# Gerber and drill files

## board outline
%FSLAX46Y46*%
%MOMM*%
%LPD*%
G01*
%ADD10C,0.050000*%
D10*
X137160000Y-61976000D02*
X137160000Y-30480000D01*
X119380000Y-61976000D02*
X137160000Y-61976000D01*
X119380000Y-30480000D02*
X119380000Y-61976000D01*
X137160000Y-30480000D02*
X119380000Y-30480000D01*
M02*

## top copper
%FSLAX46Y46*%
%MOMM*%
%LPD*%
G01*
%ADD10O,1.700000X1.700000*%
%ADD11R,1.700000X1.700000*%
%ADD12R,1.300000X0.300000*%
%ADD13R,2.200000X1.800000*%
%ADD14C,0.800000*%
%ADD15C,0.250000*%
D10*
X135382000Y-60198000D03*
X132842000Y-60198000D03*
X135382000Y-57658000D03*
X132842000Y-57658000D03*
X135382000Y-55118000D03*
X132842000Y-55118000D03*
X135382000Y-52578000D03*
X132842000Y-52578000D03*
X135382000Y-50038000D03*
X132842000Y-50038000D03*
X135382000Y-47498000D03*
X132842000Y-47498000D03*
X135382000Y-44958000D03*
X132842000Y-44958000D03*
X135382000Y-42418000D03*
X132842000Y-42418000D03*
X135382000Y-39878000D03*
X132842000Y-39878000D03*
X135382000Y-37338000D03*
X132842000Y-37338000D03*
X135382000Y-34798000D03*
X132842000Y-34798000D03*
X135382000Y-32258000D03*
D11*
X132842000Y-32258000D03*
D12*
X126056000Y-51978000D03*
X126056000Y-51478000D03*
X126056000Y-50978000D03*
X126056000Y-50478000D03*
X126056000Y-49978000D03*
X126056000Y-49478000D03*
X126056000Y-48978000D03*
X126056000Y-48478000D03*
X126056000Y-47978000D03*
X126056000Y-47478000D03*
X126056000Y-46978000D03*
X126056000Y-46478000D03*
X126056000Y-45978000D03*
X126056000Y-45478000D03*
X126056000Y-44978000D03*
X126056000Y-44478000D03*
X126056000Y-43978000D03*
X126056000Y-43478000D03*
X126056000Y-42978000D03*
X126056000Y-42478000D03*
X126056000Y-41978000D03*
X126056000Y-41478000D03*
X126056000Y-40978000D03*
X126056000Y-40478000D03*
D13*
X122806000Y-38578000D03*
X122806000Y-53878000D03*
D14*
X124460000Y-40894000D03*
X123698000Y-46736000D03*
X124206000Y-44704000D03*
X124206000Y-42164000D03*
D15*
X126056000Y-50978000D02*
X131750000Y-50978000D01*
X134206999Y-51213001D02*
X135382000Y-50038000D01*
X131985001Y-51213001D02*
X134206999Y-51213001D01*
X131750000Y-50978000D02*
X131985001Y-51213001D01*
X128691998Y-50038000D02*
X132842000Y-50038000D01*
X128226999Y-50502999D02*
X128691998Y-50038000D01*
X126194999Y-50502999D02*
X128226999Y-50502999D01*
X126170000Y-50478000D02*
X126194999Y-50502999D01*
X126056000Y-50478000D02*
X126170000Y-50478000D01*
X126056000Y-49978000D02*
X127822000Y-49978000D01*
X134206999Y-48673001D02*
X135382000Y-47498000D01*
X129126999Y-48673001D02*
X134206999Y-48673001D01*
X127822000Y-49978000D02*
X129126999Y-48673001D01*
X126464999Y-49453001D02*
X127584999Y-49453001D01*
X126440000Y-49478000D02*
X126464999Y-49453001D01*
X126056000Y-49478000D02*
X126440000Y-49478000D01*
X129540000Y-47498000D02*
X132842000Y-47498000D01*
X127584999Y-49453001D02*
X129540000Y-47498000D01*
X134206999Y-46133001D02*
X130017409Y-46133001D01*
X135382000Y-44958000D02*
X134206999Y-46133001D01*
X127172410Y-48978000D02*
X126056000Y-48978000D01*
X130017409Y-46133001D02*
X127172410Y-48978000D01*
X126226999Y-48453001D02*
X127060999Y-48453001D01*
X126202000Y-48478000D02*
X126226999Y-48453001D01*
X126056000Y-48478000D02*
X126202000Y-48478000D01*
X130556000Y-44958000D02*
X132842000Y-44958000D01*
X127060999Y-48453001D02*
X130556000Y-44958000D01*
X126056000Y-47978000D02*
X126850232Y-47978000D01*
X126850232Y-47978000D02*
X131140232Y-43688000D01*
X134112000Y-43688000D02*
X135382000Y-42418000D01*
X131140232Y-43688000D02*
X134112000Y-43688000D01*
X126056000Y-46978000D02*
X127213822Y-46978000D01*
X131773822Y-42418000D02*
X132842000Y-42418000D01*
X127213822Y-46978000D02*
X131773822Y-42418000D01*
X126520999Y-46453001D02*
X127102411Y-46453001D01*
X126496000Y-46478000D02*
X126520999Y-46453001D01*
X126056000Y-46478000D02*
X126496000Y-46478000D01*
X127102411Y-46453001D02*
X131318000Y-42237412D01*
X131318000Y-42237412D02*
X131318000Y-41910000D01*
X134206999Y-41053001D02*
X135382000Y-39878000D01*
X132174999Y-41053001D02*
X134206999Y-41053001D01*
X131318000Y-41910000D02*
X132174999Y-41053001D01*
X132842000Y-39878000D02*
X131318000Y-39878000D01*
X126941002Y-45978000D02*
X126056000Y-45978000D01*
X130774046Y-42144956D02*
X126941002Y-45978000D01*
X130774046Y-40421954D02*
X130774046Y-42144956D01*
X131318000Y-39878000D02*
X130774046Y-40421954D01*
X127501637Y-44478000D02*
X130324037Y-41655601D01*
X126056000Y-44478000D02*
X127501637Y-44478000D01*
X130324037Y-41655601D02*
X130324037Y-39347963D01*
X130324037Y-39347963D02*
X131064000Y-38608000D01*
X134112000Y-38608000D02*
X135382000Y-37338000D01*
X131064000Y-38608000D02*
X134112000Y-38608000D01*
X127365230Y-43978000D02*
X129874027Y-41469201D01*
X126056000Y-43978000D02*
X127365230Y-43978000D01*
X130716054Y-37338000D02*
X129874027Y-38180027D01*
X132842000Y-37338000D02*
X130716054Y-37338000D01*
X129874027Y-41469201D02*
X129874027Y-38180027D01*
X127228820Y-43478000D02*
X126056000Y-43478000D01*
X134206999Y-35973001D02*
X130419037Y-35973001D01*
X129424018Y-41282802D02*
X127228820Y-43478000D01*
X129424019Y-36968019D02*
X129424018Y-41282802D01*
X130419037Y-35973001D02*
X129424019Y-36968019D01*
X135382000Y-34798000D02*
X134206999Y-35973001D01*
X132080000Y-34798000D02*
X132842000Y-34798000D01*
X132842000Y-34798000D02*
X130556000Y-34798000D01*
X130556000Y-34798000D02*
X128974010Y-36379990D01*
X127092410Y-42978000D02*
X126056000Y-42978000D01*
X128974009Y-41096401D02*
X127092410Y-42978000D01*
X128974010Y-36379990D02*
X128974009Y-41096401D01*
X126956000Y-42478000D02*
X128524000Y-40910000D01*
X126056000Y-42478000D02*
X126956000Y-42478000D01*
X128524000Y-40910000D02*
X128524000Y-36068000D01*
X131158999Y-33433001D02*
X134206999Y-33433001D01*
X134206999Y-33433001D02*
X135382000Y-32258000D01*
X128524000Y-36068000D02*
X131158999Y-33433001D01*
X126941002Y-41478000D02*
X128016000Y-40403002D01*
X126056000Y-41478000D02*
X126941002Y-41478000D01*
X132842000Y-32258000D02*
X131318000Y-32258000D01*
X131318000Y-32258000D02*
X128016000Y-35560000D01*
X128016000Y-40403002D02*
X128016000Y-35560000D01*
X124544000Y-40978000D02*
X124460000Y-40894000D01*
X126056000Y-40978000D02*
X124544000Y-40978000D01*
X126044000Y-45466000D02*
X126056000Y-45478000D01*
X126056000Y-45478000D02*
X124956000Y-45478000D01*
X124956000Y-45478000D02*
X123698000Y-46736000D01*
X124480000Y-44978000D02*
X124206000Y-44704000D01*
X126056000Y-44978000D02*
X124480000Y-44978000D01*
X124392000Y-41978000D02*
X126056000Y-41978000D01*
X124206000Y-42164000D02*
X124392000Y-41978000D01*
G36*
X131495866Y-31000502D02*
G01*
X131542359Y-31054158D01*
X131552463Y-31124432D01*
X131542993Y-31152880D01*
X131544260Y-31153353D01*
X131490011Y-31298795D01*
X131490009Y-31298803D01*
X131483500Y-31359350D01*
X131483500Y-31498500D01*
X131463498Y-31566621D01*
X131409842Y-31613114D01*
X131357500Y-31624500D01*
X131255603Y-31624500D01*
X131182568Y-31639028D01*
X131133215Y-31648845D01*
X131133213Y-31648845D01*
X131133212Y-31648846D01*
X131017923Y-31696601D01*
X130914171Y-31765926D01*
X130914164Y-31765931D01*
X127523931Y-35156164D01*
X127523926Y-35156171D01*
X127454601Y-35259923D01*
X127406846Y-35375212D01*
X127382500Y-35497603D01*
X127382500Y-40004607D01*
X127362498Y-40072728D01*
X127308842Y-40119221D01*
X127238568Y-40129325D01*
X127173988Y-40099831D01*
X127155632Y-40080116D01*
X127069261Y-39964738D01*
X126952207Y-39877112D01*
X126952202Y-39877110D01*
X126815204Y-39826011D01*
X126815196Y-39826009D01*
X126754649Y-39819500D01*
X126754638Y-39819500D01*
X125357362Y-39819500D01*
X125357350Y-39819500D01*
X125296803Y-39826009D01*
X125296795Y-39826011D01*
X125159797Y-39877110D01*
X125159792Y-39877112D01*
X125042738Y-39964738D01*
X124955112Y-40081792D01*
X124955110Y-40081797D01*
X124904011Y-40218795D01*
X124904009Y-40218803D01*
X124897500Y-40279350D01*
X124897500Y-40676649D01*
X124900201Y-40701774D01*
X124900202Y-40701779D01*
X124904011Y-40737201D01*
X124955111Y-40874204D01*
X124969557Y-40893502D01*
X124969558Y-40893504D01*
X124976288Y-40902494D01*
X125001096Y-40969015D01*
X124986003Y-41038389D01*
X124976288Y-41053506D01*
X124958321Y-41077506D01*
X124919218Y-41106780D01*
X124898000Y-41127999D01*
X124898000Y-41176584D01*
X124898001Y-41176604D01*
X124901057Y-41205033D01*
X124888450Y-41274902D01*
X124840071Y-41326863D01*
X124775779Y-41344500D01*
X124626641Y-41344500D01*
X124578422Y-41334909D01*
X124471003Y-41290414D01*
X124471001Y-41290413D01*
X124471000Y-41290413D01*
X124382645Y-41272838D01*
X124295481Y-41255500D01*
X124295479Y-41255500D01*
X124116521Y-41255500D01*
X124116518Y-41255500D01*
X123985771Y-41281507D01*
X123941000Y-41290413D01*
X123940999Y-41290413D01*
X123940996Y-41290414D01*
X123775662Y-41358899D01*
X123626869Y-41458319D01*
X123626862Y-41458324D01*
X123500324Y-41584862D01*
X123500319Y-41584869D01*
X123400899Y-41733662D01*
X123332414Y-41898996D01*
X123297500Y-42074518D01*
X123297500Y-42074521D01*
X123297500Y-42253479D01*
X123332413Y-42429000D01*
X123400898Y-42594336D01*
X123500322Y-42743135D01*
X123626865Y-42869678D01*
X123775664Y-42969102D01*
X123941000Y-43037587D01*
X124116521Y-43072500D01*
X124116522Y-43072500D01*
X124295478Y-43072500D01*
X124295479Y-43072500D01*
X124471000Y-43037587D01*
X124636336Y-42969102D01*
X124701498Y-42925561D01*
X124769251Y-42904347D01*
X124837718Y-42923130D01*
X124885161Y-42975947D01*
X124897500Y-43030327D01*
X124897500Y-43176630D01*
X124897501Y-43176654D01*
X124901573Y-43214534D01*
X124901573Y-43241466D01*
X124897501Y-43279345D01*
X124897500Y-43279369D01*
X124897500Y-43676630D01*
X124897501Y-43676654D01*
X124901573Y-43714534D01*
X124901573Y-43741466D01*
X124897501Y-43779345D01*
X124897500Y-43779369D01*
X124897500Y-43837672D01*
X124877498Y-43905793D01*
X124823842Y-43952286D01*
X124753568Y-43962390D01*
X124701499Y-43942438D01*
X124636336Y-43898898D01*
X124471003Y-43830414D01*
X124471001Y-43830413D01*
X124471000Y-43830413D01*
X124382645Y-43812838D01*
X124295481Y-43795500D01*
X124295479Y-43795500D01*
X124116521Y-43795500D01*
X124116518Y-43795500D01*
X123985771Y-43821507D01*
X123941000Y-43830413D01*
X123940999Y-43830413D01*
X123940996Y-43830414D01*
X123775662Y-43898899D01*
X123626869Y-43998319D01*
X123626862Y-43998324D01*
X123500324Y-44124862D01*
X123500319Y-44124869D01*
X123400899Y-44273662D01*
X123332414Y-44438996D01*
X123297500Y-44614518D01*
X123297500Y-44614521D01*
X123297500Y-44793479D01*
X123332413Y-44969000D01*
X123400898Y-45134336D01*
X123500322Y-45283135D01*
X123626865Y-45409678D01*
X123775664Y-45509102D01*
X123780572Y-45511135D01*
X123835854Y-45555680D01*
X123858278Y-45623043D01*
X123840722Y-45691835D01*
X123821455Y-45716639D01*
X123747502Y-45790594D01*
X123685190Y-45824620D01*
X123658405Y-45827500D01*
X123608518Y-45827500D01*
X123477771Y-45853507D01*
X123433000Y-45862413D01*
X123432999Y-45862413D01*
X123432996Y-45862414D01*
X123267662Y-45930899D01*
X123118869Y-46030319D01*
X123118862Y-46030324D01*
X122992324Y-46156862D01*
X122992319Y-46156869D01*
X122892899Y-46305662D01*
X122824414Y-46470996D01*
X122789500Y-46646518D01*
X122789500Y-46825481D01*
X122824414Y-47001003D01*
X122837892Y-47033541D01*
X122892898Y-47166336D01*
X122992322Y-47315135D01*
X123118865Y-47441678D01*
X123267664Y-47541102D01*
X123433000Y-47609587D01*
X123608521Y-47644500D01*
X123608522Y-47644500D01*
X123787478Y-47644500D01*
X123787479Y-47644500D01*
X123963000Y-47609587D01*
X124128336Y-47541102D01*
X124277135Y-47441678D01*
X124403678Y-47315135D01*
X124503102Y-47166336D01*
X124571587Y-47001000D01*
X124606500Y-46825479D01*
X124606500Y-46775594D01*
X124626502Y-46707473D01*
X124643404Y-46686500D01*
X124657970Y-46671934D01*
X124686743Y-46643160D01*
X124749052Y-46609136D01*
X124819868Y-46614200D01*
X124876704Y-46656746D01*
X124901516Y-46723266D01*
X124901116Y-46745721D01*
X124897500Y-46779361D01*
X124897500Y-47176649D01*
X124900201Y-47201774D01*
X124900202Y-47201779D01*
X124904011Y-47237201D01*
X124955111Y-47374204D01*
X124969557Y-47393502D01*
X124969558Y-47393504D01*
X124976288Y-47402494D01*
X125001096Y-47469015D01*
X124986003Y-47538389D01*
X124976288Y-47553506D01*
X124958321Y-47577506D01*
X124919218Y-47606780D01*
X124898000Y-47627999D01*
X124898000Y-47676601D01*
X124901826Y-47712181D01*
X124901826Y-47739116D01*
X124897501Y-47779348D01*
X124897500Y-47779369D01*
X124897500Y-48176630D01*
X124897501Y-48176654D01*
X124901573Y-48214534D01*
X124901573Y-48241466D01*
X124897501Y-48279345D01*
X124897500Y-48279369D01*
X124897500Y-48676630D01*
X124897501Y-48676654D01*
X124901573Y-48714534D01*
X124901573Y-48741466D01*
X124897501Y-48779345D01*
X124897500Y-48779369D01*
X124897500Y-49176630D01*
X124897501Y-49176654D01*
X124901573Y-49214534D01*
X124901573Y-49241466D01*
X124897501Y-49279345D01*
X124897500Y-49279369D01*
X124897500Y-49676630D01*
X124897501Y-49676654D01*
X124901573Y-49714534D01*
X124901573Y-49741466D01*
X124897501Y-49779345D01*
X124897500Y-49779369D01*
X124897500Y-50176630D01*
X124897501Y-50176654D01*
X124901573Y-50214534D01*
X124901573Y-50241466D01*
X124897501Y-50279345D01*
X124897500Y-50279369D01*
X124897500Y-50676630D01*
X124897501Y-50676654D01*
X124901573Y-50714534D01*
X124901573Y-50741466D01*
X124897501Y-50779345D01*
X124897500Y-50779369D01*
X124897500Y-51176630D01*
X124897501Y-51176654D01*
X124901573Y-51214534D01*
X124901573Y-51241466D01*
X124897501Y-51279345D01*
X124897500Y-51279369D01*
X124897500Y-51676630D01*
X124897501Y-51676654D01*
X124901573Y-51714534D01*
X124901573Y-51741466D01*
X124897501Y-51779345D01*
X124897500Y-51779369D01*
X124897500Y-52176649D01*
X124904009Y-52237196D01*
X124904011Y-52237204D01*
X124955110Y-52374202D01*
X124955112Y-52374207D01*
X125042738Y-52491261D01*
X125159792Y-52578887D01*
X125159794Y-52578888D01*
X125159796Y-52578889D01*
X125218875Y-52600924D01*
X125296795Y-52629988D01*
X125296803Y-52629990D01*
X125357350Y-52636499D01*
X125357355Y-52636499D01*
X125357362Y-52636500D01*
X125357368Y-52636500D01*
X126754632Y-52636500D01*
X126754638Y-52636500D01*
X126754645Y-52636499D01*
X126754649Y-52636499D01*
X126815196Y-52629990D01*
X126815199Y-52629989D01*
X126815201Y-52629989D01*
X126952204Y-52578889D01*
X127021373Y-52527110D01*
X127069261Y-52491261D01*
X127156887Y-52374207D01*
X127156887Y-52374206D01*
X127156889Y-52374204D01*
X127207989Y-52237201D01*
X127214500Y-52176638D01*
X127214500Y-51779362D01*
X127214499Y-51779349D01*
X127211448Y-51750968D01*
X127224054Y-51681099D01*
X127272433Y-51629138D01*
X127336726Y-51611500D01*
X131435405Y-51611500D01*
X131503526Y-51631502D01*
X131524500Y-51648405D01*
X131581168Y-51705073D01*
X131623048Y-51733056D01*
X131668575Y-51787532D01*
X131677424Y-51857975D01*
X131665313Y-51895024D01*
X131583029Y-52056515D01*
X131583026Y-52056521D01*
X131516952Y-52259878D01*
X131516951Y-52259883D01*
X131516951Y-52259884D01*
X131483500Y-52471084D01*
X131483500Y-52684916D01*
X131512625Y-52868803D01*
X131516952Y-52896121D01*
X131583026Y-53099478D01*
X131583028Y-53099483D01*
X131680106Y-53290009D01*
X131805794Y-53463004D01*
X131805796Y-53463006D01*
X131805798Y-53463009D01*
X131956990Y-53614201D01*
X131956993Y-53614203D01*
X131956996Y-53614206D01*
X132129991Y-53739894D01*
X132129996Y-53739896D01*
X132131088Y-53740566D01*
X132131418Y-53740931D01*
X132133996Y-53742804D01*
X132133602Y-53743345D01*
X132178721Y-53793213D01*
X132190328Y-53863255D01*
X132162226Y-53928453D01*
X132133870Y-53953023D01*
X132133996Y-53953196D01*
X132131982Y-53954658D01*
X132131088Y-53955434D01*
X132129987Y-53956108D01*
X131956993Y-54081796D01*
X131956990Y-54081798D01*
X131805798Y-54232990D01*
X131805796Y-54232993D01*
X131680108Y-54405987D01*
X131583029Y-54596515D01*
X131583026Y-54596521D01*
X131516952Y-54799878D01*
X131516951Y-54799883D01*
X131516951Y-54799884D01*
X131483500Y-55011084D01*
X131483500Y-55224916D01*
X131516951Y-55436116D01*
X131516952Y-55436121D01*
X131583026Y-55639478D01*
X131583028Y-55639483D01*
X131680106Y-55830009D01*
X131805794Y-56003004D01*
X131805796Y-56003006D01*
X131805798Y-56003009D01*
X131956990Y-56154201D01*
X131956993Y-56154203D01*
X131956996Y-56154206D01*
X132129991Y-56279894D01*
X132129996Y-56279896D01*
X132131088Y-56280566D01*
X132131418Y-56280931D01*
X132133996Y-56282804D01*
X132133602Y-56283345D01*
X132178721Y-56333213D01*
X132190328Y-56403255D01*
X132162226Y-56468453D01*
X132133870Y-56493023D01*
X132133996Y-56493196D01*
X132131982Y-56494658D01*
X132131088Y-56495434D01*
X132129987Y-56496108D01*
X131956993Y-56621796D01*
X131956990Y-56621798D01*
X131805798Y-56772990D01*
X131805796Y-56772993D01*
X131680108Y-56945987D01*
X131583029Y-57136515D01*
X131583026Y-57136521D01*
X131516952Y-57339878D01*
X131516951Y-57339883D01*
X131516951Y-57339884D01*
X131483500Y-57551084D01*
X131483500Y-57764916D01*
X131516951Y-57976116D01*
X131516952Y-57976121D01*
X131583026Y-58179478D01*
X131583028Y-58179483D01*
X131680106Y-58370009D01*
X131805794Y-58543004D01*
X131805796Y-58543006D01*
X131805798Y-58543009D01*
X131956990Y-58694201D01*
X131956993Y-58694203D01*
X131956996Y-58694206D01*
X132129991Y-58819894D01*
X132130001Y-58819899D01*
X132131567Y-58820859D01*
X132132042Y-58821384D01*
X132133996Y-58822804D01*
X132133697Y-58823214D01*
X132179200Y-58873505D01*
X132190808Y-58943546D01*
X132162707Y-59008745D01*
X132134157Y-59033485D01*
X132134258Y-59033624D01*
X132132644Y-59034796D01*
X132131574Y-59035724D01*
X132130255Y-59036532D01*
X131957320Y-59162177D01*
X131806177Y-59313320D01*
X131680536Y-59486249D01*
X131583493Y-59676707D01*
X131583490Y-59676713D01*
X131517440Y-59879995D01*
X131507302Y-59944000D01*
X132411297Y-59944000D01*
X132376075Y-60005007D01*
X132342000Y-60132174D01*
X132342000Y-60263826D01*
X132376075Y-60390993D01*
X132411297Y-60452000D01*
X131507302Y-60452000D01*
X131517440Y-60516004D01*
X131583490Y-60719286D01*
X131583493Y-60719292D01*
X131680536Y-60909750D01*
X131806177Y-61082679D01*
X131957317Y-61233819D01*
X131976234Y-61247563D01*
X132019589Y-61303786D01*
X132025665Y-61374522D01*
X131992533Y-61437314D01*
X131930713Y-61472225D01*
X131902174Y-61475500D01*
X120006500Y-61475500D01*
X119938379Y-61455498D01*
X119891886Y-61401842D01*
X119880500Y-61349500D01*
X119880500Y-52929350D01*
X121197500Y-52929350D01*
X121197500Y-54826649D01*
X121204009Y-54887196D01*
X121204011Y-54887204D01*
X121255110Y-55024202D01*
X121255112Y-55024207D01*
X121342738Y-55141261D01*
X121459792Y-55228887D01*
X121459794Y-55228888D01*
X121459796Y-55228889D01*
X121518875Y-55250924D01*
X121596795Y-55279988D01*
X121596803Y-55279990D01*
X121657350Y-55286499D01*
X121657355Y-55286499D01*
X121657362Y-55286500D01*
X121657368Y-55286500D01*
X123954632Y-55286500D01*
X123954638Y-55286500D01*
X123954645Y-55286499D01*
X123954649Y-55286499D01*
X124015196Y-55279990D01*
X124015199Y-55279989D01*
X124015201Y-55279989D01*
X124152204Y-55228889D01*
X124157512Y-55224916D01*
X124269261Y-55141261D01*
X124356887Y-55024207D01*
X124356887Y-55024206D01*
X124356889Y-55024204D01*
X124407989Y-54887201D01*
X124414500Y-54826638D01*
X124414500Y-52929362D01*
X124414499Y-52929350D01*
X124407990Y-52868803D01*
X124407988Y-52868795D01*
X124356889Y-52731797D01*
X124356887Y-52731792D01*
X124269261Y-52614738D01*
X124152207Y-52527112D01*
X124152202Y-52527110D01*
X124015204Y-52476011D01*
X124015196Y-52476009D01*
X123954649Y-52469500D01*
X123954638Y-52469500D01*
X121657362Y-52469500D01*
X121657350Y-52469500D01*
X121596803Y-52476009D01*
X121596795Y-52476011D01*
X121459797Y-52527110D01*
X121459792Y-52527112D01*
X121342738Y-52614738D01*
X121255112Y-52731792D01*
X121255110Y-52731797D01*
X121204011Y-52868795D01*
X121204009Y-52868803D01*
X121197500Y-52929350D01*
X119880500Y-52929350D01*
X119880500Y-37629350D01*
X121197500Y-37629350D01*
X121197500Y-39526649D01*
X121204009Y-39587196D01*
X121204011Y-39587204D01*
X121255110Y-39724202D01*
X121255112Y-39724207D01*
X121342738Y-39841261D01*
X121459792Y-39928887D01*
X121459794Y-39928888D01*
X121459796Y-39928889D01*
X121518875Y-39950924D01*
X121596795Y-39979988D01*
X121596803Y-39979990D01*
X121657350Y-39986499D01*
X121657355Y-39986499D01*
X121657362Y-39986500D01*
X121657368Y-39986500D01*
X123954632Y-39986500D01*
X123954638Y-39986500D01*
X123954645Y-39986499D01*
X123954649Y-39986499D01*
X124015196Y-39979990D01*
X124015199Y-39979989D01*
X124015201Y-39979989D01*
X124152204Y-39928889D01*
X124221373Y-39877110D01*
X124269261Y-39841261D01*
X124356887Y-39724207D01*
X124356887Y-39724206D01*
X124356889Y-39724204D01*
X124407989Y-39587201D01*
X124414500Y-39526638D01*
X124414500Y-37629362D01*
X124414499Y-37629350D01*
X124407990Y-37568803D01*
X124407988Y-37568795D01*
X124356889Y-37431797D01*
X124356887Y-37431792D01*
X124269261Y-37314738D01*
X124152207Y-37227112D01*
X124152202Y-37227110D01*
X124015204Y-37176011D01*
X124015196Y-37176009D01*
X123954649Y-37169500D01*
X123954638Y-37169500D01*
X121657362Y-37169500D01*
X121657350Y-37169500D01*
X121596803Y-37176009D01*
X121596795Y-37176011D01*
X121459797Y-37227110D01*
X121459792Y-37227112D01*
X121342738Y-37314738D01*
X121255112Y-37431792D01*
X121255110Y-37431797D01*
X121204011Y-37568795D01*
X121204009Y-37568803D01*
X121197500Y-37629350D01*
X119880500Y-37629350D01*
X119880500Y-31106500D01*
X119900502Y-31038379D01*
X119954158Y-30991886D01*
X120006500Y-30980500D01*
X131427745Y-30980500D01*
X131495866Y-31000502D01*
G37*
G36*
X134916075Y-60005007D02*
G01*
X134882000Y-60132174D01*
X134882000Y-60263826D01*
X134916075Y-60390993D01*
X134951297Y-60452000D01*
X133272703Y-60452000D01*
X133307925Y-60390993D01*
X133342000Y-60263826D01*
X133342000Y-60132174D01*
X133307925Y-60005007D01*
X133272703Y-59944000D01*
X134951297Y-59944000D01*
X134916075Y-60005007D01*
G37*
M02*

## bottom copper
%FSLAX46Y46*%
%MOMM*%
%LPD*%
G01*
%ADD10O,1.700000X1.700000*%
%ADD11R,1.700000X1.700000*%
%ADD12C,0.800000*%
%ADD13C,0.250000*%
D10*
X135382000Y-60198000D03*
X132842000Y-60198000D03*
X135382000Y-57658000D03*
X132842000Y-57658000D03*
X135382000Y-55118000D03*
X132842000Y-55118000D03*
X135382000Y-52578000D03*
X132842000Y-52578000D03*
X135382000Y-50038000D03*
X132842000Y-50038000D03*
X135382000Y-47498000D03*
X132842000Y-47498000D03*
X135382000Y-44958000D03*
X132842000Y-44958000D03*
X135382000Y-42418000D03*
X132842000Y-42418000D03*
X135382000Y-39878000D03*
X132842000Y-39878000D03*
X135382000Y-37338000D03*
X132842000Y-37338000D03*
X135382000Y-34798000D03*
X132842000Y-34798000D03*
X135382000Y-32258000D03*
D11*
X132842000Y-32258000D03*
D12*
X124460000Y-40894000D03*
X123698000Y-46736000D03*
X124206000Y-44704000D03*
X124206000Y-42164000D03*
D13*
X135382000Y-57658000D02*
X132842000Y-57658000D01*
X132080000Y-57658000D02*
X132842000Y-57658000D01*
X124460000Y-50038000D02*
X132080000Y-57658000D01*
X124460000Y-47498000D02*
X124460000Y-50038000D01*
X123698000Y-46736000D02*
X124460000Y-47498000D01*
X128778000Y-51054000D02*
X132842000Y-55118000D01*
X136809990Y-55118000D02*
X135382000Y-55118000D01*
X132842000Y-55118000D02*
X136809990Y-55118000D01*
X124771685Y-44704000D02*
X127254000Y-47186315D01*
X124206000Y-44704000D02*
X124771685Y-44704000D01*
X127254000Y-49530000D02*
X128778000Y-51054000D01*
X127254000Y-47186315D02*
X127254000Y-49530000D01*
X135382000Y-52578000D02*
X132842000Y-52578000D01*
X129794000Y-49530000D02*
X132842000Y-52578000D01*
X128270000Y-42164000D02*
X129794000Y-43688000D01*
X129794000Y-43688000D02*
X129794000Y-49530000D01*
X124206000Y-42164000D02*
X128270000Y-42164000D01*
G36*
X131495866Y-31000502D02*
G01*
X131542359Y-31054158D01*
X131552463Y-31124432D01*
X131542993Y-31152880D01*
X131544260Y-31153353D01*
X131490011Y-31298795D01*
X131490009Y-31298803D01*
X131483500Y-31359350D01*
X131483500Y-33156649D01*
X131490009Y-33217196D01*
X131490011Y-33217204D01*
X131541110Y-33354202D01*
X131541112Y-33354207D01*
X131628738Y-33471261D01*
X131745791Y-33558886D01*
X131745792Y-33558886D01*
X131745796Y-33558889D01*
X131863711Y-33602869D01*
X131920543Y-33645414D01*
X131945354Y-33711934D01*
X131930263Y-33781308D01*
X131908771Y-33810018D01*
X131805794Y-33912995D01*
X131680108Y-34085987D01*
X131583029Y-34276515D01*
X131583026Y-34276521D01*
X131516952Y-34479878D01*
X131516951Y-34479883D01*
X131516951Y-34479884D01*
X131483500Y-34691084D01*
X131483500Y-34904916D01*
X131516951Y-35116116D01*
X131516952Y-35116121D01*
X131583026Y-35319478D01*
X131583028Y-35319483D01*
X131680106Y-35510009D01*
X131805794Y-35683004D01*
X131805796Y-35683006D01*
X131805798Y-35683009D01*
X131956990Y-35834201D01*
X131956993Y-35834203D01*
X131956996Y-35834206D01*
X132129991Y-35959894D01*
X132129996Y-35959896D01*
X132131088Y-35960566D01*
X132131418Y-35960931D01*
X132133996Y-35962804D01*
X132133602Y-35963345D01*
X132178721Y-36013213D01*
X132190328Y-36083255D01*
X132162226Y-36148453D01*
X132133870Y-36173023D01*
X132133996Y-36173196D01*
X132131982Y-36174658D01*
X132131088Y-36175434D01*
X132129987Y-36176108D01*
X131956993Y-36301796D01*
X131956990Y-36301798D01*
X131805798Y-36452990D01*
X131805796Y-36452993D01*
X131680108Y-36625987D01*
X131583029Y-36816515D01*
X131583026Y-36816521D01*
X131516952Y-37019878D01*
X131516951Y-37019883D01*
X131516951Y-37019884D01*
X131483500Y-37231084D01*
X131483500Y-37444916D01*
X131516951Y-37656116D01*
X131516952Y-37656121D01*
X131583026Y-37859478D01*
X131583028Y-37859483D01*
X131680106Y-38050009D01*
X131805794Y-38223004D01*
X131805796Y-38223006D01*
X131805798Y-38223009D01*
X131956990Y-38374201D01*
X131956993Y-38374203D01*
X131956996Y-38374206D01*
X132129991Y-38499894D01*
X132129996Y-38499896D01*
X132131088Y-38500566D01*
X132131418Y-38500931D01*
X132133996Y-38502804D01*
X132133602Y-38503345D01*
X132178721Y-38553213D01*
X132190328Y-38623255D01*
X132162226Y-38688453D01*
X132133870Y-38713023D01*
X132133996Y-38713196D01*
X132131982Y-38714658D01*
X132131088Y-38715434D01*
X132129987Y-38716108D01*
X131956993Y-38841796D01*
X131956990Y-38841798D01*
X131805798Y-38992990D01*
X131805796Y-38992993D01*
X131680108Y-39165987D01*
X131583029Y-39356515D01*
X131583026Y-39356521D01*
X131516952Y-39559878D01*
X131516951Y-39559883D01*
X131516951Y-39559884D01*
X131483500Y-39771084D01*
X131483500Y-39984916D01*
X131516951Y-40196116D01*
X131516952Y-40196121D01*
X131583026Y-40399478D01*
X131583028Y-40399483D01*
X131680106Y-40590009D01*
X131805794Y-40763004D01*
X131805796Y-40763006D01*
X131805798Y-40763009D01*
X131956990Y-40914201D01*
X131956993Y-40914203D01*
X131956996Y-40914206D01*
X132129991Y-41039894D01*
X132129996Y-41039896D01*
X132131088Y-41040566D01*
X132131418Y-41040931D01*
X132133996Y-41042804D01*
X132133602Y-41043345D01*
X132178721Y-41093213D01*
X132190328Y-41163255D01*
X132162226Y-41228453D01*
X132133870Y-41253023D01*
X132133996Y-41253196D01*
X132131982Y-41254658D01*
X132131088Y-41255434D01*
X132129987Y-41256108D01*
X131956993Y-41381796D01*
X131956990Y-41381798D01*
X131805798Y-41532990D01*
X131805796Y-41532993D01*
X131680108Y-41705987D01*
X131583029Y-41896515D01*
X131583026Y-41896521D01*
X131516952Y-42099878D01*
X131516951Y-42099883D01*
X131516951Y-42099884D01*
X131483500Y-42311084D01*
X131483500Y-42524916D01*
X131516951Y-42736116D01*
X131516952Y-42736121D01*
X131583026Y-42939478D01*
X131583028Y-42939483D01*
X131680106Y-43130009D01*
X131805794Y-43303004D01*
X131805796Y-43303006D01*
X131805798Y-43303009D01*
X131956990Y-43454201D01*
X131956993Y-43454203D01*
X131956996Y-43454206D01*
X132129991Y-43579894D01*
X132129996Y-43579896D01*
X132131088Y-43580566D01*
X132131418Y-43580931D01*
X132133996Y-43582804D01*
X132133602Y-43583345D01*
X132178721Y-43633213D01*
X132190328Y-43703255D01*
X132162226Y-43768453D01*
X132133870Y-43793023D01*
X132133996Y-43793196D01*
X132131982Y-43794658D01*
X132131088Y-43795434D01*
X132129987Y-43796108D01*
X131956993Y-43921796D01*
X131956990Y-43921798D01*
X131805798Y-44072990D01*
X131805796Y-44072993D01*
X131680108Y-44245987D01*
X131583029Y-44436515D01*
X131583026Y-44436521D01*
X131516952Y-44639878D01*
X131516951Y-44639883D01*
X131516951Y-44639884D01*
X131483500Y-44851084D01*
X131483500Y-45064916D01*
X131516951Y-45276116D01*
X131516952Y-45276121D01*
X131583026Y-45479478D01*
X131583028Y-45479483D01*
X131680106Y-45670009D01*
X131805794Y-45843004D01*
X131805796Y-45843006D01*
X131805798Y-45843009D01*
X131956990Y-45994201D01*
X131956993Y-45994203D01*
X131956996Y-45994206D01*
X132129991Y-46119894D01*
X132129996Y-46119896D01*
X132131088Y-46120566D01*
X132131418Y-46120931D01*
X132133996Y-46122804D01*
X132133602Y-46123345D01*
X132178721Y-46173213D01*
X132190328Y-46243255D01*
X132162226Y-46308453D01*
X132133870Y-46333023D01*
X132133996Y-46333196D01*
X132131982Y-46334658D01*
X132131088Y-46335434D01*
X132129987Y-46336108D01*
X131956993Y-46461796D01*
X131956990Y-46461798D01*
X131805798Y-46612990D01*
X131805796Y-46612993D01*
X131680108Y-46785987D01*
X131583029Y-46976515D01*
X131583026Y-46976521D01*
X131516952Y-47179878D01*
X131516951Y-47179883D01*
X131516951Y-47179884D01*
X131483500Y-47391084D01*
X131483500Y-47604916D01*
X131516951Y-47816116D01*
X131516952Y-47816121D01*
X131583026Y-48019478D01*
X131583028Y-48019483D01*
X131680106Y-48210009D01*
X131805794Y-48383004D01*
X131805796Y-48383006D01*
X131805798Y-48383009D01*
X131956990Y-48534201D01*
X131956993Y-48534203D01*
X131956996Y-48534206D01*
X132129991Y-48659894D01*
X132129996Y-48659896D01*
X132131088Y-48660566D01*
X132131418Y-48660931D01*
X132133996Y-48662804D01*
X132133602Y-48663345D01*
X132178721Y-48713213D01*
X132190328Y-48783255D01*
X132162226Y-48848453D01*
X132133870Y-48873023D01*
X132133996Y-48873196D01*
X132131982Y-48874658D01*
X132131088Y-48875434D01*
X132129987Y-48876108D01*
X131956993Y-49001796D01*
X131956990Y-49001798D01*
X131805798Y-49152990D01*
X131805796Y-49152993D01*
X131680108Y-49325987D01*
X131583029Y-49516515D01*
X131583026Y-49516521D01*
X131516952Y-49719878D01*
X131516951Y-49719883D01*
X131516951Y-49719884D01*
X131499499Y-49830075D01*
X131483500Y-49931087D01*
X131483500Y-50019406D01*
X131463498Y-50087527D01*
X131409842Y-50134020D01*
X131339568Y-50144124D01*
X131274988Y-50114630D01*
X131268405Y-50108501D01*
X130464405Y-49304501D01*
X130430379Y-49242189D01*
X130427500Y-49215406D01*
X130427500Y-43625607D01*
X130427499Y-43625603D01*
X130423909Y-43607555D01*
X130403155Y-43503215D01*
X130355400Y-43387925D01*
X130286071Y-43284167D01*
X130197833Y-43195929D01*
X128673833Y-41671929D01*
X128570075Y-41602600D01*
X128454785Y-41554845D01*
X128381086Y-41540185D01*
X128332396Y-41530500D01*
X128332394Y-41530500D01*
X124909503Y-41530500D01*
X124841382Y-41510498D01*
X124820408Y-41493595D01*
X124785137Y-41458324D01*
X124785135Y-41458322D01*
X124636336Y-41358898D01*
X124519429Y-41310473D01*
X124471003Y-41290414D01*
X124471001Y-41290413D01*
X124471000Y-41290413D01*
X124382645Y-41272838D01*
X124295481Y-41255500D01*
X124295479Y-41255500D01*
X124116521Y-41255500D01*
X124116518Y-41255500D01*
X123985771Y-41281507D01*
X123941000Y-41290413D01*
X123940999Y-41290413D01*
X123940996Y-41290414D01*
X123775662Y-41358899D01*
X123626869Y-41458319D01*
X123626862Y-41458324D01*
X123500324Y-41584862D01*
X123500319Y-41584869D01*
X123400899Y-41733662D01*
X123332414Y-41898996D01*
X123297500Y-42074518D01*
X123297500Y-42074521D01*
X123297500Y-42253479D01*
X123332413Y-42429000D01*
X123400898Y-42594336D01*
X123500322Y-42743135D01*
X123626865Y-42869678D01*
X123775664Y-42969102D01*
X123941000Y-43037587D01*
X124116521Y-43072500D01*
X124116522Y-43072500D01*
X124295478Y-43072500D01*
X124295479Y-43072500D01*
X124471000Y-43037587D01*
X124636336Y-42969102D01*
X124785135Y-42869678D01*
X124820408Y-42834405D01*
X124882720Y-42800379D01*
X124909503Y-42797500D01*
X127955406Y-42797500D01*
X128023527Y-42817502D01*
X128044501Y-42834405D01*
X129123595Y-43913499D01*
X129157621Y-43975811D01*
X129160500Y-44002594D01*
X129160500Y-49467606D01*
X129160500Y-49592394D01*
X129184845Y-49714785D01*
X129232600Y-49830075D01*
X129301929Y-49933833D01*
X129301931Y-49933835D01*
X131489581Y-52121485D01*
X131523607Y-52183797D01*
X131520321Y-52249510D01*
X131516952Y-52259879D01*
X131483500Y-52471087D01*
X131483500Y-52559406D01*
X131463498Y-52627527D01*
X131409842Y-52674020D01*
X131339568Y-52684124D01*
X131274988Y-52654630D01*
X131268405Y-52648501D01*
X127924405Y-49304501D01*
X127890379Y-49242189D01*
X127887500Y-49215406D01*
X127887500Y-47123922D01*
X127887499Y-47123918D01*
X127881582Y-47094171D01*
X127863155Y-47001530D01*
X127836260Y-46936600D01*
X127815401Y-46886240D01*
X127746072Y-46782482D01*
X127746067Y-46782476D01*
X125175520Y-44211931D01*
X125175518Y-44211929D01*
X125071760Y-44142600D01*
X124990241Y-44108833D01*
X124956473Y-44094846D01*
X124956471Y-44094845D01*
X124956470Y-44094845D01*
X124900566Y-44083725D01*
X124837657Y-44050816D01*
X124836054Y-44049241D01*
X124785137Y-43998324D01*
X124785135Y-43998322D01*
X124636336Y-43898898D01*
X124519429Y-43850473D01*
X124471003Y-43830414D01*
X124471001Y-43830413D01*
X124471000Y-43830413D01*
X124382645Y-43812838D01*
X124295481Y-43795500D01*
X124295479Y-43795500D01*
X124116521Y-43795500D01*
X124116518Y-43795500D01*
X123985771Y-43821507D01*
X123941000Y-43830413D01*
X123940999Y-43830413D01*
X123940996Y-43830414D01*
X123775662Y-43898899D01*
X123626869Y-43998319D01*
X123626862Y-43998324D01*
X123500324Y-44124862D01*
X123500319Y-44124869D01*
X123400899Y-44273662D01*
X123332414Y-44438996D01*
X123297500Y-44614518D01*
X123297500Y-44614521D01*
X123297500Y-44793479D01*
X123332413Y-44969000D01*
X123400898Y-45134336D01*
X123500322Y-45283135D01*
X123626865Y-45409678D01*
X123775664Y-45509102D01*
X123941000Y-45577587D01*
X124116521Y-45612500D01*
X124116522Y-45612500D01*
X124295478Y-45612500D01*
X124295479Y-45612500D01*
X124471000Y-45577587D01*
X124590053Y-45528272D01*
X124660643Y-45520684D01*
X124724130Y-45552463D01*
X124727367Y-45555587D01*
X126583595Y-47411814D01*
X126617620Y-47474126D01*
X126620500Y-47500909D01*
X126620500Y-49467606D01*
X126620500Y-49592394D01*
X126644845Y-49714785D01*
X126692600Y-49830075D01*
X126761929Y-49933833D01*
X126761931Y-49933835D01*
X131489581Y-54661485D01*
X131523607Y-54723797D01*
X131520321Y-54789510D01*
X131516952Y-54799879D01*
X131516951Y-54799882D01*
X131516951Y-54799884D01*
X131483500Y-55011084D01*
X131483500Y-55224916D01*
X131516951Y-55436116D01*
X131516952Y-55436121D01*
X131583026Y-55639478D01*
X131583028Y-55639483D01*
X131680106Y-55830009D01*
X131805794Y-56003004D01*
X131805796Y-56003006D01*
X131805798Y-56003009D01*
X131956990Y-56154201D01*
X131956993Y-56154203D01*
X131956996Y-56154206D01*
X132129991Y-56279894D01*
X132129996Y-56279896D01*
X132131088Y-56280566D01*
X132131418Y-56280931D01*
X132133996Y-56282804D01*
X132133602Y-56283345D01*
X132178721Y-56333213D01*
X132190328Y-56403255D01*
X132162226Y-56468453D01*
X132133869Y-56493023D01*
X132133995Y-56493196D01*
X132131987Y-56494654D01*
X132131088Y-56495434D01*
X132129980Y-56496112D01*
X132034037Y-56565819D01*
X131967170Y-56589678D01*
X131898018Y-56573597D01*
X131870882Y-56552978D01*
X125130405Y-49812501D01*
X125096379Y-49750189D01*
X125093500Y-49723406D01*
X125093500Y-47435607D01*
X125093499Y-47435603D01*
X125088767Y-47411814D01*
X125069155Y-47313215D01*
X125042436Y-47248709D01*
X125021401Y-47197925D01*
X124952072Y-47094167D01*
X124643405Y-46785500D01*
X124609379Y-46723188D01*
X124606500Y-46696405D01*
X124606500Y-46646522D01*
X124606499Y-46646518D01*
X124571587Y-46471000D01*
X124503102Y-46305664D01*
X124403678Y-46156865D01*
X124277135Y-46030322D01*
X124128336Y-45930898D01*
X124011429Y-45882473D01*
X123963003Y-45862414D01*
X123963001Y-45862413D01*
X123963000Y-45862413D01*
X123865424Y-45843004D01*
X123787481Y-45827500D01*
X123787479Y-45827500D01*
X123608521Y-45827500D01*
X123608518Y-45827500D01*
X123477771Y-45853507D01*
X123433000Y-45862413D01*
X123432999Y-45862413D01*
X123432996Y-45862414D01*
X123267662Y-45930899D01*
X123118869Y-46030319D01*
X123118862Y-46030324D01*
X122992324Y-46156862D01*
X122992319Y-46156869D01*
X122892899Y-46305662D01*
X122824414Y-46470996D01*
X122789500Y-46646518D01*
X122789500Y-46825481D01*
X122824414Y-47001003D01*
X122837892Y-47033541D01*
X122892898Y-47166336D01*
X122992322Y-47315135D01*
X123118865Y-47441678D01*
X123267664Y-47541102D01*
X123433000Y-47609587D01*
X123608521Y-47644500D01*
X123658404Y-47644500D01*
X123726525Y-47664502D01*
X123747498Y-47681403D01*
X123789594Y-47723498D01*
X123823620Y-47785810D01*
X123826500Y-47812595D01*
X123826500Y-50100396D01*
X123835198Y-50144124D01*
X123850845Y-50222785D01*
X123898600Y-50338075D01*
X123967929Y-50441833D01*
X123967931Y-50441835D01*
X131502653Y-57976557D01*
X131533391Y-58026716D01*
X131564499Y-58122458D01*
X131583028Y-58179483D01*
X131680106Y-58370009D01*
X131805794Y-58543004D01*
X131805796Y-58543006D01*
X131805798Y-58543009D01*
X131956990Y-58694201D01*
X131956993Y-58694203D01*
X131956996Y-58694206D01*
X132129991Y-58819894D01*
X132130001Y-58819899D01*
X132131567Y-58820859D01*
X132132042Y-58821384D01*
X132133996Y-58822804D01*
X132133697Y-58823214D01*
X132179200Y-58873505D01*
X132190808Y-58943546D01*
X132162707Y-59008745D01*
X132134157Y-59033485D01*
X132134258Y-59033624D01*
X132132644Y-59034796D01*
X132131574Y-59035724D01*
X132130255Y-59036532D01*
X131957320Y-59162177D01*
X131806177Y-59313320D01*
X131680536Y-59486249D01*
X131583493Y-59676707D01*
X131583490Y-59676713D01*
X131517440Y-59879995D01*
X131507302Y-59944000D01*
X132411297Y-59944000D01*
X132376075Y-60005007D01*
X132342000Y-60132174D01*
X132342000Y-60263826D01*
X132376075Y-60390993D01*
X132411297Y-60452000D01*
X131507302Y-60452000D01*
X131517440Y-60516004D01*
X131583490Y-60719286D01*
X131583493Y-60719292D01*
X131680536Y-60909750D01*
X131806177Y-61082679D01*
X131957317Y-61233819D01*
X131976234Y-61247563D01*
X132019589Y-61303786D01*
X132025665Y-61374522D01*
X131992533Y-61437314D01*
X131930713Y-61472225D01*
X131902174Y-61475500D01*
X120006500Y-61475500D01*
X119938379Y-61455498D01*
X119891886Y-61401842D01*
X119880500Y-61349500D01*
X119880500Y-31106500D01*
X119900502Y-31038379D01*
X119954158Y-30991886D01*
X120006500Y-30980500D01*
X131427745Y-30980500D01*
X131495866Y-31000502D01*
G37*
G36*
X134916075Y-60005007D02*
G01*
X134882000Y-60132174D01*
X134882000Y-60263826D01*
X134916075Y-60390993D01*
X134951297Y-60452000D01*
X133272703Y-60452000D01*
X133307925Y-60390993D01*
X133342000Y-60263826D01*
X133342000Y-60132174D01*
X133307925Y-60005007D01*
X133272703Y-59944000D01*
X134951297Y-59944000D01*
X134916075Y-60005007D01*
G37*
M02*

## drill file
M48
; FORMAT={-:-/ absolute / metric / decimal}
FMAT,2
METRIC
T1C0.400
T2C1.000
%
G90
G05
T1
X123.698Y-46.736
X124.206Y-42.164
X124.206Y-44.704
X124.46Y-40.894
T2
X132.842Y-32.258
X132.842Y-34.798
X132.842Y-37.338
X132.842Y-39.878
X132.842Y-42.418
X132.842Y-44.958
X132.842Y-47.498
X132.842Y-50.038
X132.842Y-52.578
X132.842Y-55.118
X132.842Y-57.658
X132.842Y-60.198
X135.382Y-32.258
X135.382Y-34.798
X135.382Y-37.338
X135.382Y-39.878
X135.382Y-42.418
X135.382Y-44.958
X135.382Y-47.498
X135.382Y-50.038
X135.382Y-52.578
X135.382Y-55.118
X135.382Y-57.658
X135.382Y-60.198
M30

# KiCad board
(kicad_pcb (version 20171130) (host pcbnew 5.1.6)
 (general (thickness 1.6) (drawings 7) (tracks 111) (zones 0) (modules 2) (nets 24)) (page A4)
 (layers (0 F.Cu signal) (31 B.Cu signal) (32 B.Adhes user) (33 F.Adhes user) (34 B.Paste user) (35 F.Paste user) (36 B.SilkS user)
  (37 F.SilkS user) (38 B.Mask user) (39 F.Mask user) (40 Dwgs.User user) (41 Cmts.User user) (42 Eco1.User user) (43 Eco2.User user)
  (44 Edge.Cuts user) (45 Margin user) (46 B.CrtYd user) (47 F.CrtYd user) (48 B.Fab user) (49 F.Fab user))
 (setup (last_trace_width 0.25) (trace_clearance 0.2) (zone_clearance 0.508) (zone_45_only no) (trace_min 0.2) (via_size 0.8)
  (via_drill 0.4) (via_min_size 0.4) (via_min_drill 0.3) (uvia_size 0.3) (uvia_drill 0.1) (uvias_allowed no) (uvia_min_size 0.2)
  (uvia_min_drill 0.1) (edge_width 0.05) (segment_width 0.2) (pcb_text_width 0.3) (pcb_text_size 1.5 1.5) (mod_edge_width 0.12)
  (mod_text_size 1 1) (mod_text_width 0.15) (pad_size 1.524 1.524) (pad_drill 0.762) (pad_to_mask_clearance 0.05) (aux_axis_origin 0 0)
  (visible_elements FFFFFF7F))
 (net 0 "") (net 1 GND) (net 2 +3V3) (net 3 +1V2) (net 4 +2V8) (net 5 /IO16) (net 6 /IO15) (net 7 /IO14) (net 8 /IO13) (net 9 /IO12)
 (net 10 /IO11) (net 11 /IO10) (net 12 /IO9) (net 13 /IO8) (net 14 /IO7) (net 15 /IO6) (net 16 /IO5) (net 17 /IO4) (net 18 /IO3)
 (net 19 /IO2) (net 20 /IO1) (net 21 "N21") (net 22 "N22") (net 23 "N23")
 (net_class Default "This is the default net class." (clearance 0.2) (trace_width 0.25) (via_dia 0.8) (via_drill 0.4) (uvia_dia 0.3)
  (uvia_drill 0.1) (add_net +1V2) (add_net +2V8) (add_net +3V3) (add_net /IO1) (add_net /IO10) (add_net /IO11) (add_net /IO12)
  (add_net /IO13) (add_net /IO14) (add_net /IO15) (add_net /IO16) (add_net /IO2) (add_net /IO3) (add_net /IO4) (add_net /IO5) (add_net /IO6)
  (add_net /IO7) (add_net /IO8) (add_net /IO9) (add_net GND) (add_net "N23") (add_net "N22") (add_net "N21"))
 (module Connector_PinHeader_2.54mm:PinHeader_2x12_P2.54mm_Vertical (layer F.Cu) (at 132.842 32.258)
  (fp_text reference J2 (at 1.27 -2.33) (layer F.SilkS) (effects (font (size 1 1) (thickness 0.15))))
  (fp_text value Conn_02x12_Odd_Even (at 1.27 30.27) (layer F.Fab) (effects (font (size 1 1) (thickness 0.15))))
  (pad 24 thru_hole oval (at 2.54 27.94) (size 1.7 1.7) (drill 1) (layers *.Cu *.Mask) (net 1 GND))
  (pad 23 thru_hole oval (at 0 27.94) (size 1.7 1.7) (drill 1) (layers *.Cu *.Mask) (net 1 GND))
  (pad 22 thru_hole oval (at 2.54 25.4) (size 1.7 1.7) (drill 1) (layers *.Cu *.Mask) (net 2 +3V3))
  (pad 21 thru_hole oval (at 0 25.4) (size 1.7 1.7) (drill 1) (layers *.Cu *.Mask) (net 2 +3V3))
  (pad 20 thru_hole oval (at 2.54 22.86) (size 1.7 1.7) (drill 1) (layers *.Cu *.Mask) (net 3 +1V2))
  (pad 19 thru_hole oval (at 0 22.86) (size 1.7 1.7) (drill 1) (layers *.Cu *.Mask) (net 3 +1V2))
  (pad 18 thru_hole oval (at 2.54 20.32) (size 1.7 1.7) (drill 1) (layers *.Cu *.Mask) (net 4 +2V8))
  (pad 17 thru_hole oval (at 0 20.32) (size 1.7 1.7) (drill 1) (layers *.Cu *.Mask) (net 4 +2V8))
  (pad 16 thru_hole oval (at 2.54 17.78) (size 1.7 1.7) (drill 1) (layers *.Cu *.Mask) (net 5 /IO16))
  (pad 15 thru_hole oval (at 0 17.78) (size 1.7 1.7) (drill 1) (layers *.Cu *.Mask) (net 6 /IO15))
  (pad 14 thru_hole oval (at 2.54 15.24) (size 1.7 1.7) (drill 1) (layers *.Cu *.Mask) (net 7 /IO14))
  (pad 13 thru_hole oval (at 0 15.24) (size 1.7 1.7) (drill 1) (layers *.Cu *.Mask) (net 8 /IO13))
  (pad 12 thru_hole oval (at 2.54 12.7) (size 1.7 1.7) (drill 1) (layers *.Cu *.Mask) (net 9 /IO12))
  (pad 11 thru_hole oval (at 0 12.7) (size 1.7 1.7) (drill 1) (layers *.Cu *.Mask) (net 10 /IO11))
  (pad 10 thru_hole oval (at 2.54 10.16) (size 1.7 1.7) (drill 1) (layers *.Cu *.Mask) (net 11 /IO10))
  (pad 9 thru_hole oval (at 0 10.16) (size 1.7 1.7) (drill 1) (layers *.Cu *.Mask) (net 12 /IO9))
  (pad 8 thru_hole oval (at 2.54 7.62) (size 1.7 1.7) (drill 1) (layers *.Cu *.Mask) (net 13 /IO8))
  (pad 7 thru_hole oval (at 0 7.62) (size 1.7 1.7) (drill 1) (layers *.Cu *.Mask) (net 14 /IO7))
  (pad 6 thru_hole oval (at 2.54 5.08) (size 1.7 1.7) (drill 1) (layers *.Cu *.Mask) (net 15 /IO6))
  (pad 5 thru_hole oval (at 0 5.08) (size 1.7 1.7) (drill 1) (layers *.Cu *.Mask) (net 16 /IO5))
  (pad 4 thru_hole oval (at 2.54 2.54) (size 1.7 1.7) (drill 1) (layers *.Cu *.Mask) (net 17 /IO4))
  (pad 3 thru_hole oval (at 0 2.54) (size 1.7 1.7) (drill 1) (layers *.Cu *.Mask) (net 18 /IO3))
  (pad 2 thru_hole oval (at 2.54 0) (size 1.7 1.7) (drill 1) (layers *.Cu *.Mask) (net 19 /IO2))
  (pad 1 thru_hole rect (at 0 0) (size 1.7 1.7) (drill 1) (layers *.Cu *.Mask) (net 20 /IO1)))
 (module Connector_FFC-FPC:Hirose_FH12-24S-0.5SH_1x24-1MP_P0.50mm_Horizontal (layer F.Cu) (at 124.206 46.228 270)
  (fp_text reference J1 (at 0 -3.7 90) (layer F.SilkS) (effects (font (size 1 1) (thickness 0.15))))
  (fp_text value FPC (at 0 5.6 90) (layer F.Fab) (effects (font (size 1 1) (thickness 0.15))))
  (pad 24 smd rect (at 5.75 -1.85 270) (size 0.3 1.3) (layers F.Cu F.Paste F.Mask) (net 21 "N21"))
  (pad 23 smd rect (at 5.25 -1.85 270) (size 0.3 1.3) (layers F.Cu F.Paste F.Mask) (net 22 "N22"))
  (pad 22 smd rect (at 4.75 -1.85 270) (size 0.3 1.3) (layers F.Cu F.Paste F.Mask) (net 5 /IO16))
  (pad 21 smd rect (at 4.25 -1.85 270) (size 0.3 1.3) (layers F.Cu F.Paste F.Mask) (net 6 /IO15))
  (pad 20 smd rect (at 3.75 -1.85 270) (size 0.3 1.3) (layers F.Cu F.Paste F.Mask) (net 7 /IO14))
  (pad 19 smd rect (at 3.25 -1.85 270) (size 0.3 1.3) (layers F.Cu F.Paste F.Mask) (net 8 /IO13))
  (pad 18 smd rect (at 2.75 -1.85 270) (size 0.3 1.3) (layers F.Cu F.Paste F.Mask) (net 9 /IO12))
  (pad 17 smd rect (at 2.25 -1.85 270) (size 0.3 1.3) (layers F.Cu F.Paste F.Mask) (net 10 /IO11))
  (pad 16 smd rect (at 1.75 -1.85 270) (size 0.3 1.3) (layers F.Cu F.Paste F.Mask) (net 11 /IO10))
  (pad 15 smd rect (at 1.25 -1.85 270) (size 0.3 1.3) (layers F.Cu F.Paste F.Mask) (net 1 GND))
  (pad 14 smd rect (at 0.75 -1.85 270) (size 0.3 1.3) (layers F.Cu F.Paste F.Mask) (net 12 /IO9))
  (pad 13 smd rect (at 0.25 -1.85 270) (size 0.3 1.3) (layers F.Cu F.Paste F.Mask) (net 13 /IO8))
  (pad 12 smd rect (at -0.25 -1.85 270) (size 0.3 1.3) (layers F.Cu F.Paste F.Mask) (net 14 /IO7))
  (pad 11 smd rect (at -0.75 -1.85 270) (size 0.3 1.3) (layers F.Cu F.Paste F.Mask) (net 2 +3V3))
  (pad 10 smd rect (at -1.25 -1.85 270) (size 0.3 1.3) (layers F.Cu F.Paste F.Mask) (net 3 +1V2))
  (pad 9 smd rect (at -1.75 -1.85 270) (size 0.3 1.3) (layers F.Cu F.Paste F.Mask) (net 15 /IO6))
  (pad 8 smd rect (at -2.25 -1.85 270) (size 0.3 1.3) (layers F.Cu F.Paste F.Mask) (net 16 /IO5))
  (pad 7 smd rect (at -2.75 -1.85 270) (size 0.3 1.3) (layers F.Cu F.Paste F.Mask) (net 17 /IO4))
  (pad 6 smd rect (at -3.25 -1.85 270) (size 0.3 1.3) (layers F.Cu F.Paste F.Mask) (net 18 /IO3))
  (pad 5 smd rect (at -3.75 -1.85 270) (size 0.3 1.3) (layers F.Cu F.Paste F.Mask) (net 19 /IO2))
  (pad 4 smd rect (at -4.25 -1.85 270) (size 0.3 1.3) (layers F.Cu F.Paste F.Mask) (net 4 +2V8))
  (pad 3 smd rect (at -4.75 -1.85 270) (size 0.3 1.3) (layers F.Cu F.Paste F.Mask) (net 20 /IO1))
  (pad 2 smd rect (at -5.25 -1.85 270) (size 0.3 1.3) (layers F.Cu F.Paste F.Mask) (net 1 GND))
  (pad 1 smd rect (at -5.75 -1.85 270) (size 0.3 1.3) (layers F.Cu F.Paste F.Mask) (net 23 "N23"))
  (pad MP smd rect (at -7.65 1.4 270) (size 1.8 2.2) (layers F.Cu F.Paste F.Mask))
  (pad MP smd rect (at 7.65 1.4 270) (size 1.8 2.2) (layers F.Cu F.Paste F.Mask)))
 (gr_line (start 137.16 61.976) (end 137.16 30.48) (layer Edge.Cuts) (width 0.05))
 (gr_line (start 119.38 61.976) (end 137.16 61.976) (layer Edge.Cuts) (width 0.05))
 (gr_line (start 119.38 30.48) (end 119.38 61.976) (layer Edge.Cuts) (width 0.05))
 (gr_line (start 137.16 30.48) (end 119.38 30.48) (layer Edge.Cuts) (width 0.05))
 (segment (start 126.056 50.978) (end 131.75 50.978) (width 0.25) (layer F.Cu) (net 5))
 (segment (start 134.206999 51.213001) (end 135.382 50.038) (width 0.25) (layer F.Cu) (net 5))
 (segment (start 131.985001 51.213001) (end 134.206999 51.213001) (width 0.25) (layer F.Cu) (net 5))
 (segment (start 131.75 50.978) (end 131.985001 51.213001) (width 0.25) (layer F.Cu) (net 5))
 (segment (start 128.691998 50.038) (end 132.842 50.038) (width 0.25) (layer F.Cu) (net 6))
 (segment (start 128.226999 50.502999) (end 128.691998 50.038) (width 0.25) (layer F.Cu) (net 6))
 (segment (start 126.194999 50.502999) (end 128.226999 50.502999) (width 0.25) (layer F.Cu) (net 6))
 (segment (start 126.17 50.478) (end 126.194999 50.502999) (width 0.25) (layer F.Cu) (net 6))
 (segment (start 126.056 50.478) (end 126.17 50.478) (width 0.25) (layer F.Cu) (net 6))
 (segment (start 126.056 49.978) (end 127.822 49.978) (width 0.25) (layer F.Cu) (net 7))
 (segment (start 134.206999 48.673001) (end 135.382 47.498) (width 0.25) (layer F.Cu) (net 7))
 (segment (start 129.126999 48.673001) (end 134.206999 48.673001) (width 0.25) (layer F.Cu) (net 7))
 (segment (start 127.822 49.978) (end 129.126999 48.673001) (width 0.25) (layer F.Cu) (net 7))
 (segment (start 126.464999 49.453001) (end 127.584999 49.453001) (width 0.25) (layer F.Cu) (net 8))
 (segment (start 126.44 49.478) (end 126.464999 49.453001) (width 0.25) (layer F.Cu) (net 8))
 (segment (start 126.056 49.478) (end 126.44 49.478) (width 0.25) (layer F.Cu) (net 8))
 (segment (start 129.54 47.498) (end 132.842 47.498) (width 0.25) (layer F.Cu) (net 8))
 (segment (start 127.584999 49.453001) (end 129.54 47.498) (width 0.25) (layer F.Cu) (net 8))
 (segment (start 134.206999 46.133001) (end 130.017409 46.133001) (width 0.25) (layer F.Cu) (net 9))
 (segment (start 135.382 44.958) (end 134.206999 46.133001) (width 0.25) (layer F.Cu) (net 9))
 (segment (start 127.17241 48.978) (end 126.056 48.978) (width 0.25) (layer F.Cu) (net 9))
 (segment (start 130.017409 46.133001) (end 127.17241 48.978) (width 0.25) (layer F.Cu) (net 9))
 (segment (start 126.226999 48.453001) (end 127.060999 48.453001) (width 0.25) (layer F.Cu) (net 10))
 (segment (start 126.202 48.478) (end 126.226999 48.453001) (width 0.25) (layer F.Cu) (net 10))
 (segment (start 126.056 48.478) (end 126.202 48.478) (width 0.25) (layer F.Cu) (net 10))
 (segment (start 130.556 44.958) (end 132.842 44.958) (width 0.25) (layer F.Cu) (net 10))
 (segment (start 127.060999 48.453001) (end 130.556 44.958) (width 0.25) (layer F.Cu) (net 10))
 (segment (start 126.056 47.978) (end 126.850232 47.978) (width 0.25) (layer F.Cu) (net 11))
 (segment (start 126.850232 47.978) (end 131.140232 43.688) (width 0.25) (layer F.Cu) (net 11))
 (segment (start 134.112 43.688) (end 135.382 42.418) (width 0.25) (layer F.Cu) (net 11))
 (segment (start 131.140232 43.688) (end 134.112 43.688) (width 0.25) (layer F.Cu) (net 11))
 (segment (start 126.056 46.978) (end 127.213822 46.978) (width 0.25) (layer F.Cu) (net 12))
 (segment (start 131.773822 42.418) (end 132.842 42.418) (width 0.25) (layer F.Cu) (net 12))
 (segment (start 127.213822 46.978) (end 131.773822 42.418) (width 0.25) (layer F.Cu) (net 12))
 (segment (start 126.520999 46.453001) (end 127.102411 46.453001) (width 0.25) (layer F.Cu) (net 13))
 (segment (start 126.496 46.478) (end 126.520999 46.453001) (width 0.25) (layer F.Cu) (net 13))
 (segment (start 126.056 46.478) (end 126.496 46.478) (width 0.25) (layer F.Cu) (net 13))
 (segment (start 127.102411 46.453001) (end 131.318 42.237412) (width 0.25) (layer F.Cu) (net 13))
 (segment (start 131.318 42.237412) (end 131.318 41.91) (width 0.25) (layer F.Cu) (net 13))
 (segment (start 134.206999 41.053001) (end 135.382 39.878) (width 0.25) (layer F.Cu) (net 13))
 (segment (start 132.174999 41.053001) (end 134.206999 41.053001) (width 0.25) (layer F.Cu) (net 13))
 (segment (start 131.318 41.91) (end 132.174999 41.053001) (width 0.25) (layer F.Cu) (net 13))
 (segment (start 132.842 39.878) (end 131.318 39.878) (width 0.25) (layer F.Cu) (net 14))
 (segment (start 126.941002 45.978) (end 126.056 45.978) (width 0.25) (layer F.Cu) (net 14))
 (segment (start 130.774046 42.144956) (end 126.941002 45.978) (width 0.25) (layer F.Cu) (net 14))
 (segment (start 130.774046 40.421954) (end 130.774046 42.144956) (width 0.25) (layer F.Cu) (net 14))
 (segment (start 131.318 39.878) (end 130.774046 40.421954) (width 0.25) (layer F.Cu) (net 14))
 (segment (start 127.501637 44.478) (end 130.324037 41.655601) (width 0.25) (layer F.Cu) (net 15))
 (segment (start 126.056 44.478) (end 127.501637 44.478) (width 0.25) (layer F.Cu) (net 15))
 (segment (start 130.324037 41.655601) (end 130.324037 39.347963) (width 0.25) (layer F.Cu) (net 15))
 (segment (start 130.324037 39.347963) (end 131.064 38.608) (width 0.25) (layer F.Cu) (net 15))
 (segment (start 134.112 38.608) (end 135.382 37.338) (width 0.25) (layer F.Cu) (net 15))
 (segment (start 131.064 38.608) (end 134.112 38.608) (width 0.25) (layer F.Cu) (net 15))
 (segment (start 127.36523 43.978) (end 129.874027 41.469201) (width 0.25) (layer F.Cu) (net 16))
 (segment (start 126.056 43.978) (end 127.36523 43.978) (width 0.25) (layer F.Cu) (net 16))
 (segment (start 130.716054 37.338) (end 129.874027 38.180027) (width 0.25) (layer F.Cu) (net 16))
 (segment (start 132.842 37.338) (end 130.716054 37.338) (width 0.25) (layer F.Cu) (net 16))
 (segment (start 129.874027 41.469201) (end 129.874027 38.180027) (width 0.25) (layer F.Cu) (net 16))
 (segment (start 127.22882 43.478) (end 126.056 43.478) (width 0.25) (layer F.Cu) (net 17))
 (segment (start 134.206999 35.973001) (end 130.419037 35.973001) (width 0.25) (layer F.Cu) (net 17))
 (segment (start 129.424018 41.282802) (end 127.22882 43.478) (width 0.25) (layer F.Cu) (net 17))
 (segment (start 129.424019 36.968019) (end 129.424018 41.282802) (width 0.25) (layer F.Cu) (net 17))
 (segment (start 130.419037 35.973001) (end 129.424019 36.968019) (width 0.25) (layer F.Cu) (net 17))
 (segment (start 135.382 34.798) (end 134.206999 35.973001) (width 0.25) (layer F.Cu) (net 17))
 (segment (start 132.08 34.798) (end 132.842 34.798) (width 0.25) (layer F.Cu) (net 18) (status 30))
 (segment (start 132.842 34.798) (end 130.556 34.798) (width 0.25) (layer F.Cu) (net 18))
 (segment (start 130.556 34.798) (end 128.97401 36.37999) (width 0.25) (layer F.Cu) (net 18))
 (segment (start 127.09241 42.978) (end 126.056 42.978) (width 0.25) (layer F.Cu) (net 18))
 (segment (start 128.974009 41.096401) (end 127.09241 42.978) (width 0.25) (layer F.Cu) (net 18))
 (segment (start 128.97401 36.37999) (end 128.974009 41.096401) (width 0.25) (layer F.Cu) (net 18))
 (segment (start 126.956 42.478) (end 128.524 40.91) (width 0.25) (layer F.Cu) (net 19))
 (segment (start 126.056 42.478) (end 126.956 42.478) (width 0.25) (layer F.Cu) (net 19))
 (segment (start 128.524 40.91) (end 128.524 36.068) (width 0.25) (layer F.Cu) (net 19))
 (segment (start 131.158999 33.433001) (end 134.206999 33.433001) (width 0.25) (layer F.Cu) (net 19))
 (segment (start 134.206999 33.433001) (end 135.382 32.258) (width 0.25) (layer F.Cu) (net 19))
 (segment (start 128.524 36.068) (end 131.158999 33.433001) (width 0.25) (layer F.Cu) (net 19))
 (segment (start 126.941002 41.478) (end 128.016 40.403002) (width 0.25) (layer F.Cu) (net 20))
 (segment (start 126.056 41.478) (end 126.941002 41.478) (width 0.25) (layer F.Cu) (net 20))
 (segment (start 132.842 32.258) (end 131.318 32.258) (width 0.25) (layer F.Cu) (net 20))
 (segment (start 131.318 32.258) (end 128.016 35.56) (width 0.25) (layer F.Cu) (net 20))
 (segment (start 128.016 40.403002) (end 128.016 35.56) (width 0.25) (layer F.Cu) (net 20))
 (via (at 124.46 40.894) (size 0.8) (drill 0.4) (layers F.Cu B.Cu) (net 1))
 (segment (start 124.544 40.978) (end 124.46 40.894) (width 0.25) (layer F.Cu) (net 1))
 (segment (start 126.056 40.978) (end 124.544 40.978) (width 0.25) (layer F.Cu) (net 1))
 (segment (start 126.044 45.466) (end 126.056 45.478) (width 0.25) (layer F.Cu) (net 2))
 (segment (start 135.382 57.658) (end 132.842 57.658) (width 0.25) (layer B.Cu) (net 2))
 (segment (start 126.056 45.478) (end 124.956 45.478) (width 0.25) (layer F.Cu) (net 2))
 (segment (start 132.08 57.658) (end 132.842 57.658) (width 0.25) (layer B.Cu) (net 2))
 (segment (start 124.46 50.038) (end 132.08 57.658) (width 0.25) (layer B.Cu) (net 2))
 (via (at 123.698 46.736) (size 0.8) (drill 0.4) (layers F.Cu B.Cu) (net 2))
 (segment (start 124.956 45.478) (end 123.698 46.736) (width 0.25) (layer F.Cu) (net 2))
 (segment (start 124.46 47.498) (end 124.46 50.038) (width 0.25) (layer B.Cu) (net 2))
 (segment (start 123.698 46.736) (end 124.46 47.498) (width 0.25) (layer B.Cu) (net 2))
 (via (at 124.206 44.704) (size 0.8) (drill 0.4) (layers F.Cu B.Cu) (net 3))
 (segment (start 124.48 44.978) (end 124.206 44.704) (width 0.25) (layer F.Cu) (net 3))
 (segment (start 126.056 44.978) (end 124.48 44.978) (width 0.25) (layer F.Cu) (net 3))
 (segment (start 128.778 51.054) (end 132.842 55.118) (width 0.25) (layer B.Cu) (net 3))
 (segment (start 136.80999 55.118) (end 135.382 55.118) (width 0.25) (layer B.Cu) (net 3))
 (segment (start 132.842 55.118) (end 136.80999 55.118) (width 0.25) (layer B.Cu) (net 3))
 (segment (start 124.771685 44.704) (end 127.254 47.186315) (width 0.25) (layer B.Cu) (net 3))
 (segment (start 124.206 44.704) (end 124.771685 44.704) (width 0.25) (layer B.Cu) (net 3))
 (segment (start 127.254 49.53) (end 128.778 51.054) (width 0.25) (layer B.Cu) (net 3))
 (segment (start 127.254 47.186315) (end 127.254 49.53) (width 0.25) (layer B.Cu) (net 3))
 (segment (start 135.382 52.578) (end 132.842 52.578) (width 0.25) (layer B.Cu) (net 4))
 (via (at 124.206 42.164) (size 0.8) (drill 0.4) (layers F.Cu B.Cu) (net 4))
 (segment (start 124.392 41.978) (end 126.056 41.978) (width 0.25) (layer F.Cu) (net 4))
 (segment (start 124.206 42.164) (end 124.392 41.978) (width 0.25) (layer F.Cu) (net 4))
 (segment (start 129.794 49.53) (end 132.842 52.578) (width 0.25) (layer B.Cu) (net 4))
 (segment (start 128.27 42.164) (end 129.794 43.688) (width 0.25) (layer B.Cu) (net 4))
 (segment (start 129.794 43.688) (end 129.794 49.53) (width 0.25) (layer B.Cu) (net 4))
 (segment (start 124.206 42.164) (end 128.27 42.164) (width 0.25) (layer B.Cu) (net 4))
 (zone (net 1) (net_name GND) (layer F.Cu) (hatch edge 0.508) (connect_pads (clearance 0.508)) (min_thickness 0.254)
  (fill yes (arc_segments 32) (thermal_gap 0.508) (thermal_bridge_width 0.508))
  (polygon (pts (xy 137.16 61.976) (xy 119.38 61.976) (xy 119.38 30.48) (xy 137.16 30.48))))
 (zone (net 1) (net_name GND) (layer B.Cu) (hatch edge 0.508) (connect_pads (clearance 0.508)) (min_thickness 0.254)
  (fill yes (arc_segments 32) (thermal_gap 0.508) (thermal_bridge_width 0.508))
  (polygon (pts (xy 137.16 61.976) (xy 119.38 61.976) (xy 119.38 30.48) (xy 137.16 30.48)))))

